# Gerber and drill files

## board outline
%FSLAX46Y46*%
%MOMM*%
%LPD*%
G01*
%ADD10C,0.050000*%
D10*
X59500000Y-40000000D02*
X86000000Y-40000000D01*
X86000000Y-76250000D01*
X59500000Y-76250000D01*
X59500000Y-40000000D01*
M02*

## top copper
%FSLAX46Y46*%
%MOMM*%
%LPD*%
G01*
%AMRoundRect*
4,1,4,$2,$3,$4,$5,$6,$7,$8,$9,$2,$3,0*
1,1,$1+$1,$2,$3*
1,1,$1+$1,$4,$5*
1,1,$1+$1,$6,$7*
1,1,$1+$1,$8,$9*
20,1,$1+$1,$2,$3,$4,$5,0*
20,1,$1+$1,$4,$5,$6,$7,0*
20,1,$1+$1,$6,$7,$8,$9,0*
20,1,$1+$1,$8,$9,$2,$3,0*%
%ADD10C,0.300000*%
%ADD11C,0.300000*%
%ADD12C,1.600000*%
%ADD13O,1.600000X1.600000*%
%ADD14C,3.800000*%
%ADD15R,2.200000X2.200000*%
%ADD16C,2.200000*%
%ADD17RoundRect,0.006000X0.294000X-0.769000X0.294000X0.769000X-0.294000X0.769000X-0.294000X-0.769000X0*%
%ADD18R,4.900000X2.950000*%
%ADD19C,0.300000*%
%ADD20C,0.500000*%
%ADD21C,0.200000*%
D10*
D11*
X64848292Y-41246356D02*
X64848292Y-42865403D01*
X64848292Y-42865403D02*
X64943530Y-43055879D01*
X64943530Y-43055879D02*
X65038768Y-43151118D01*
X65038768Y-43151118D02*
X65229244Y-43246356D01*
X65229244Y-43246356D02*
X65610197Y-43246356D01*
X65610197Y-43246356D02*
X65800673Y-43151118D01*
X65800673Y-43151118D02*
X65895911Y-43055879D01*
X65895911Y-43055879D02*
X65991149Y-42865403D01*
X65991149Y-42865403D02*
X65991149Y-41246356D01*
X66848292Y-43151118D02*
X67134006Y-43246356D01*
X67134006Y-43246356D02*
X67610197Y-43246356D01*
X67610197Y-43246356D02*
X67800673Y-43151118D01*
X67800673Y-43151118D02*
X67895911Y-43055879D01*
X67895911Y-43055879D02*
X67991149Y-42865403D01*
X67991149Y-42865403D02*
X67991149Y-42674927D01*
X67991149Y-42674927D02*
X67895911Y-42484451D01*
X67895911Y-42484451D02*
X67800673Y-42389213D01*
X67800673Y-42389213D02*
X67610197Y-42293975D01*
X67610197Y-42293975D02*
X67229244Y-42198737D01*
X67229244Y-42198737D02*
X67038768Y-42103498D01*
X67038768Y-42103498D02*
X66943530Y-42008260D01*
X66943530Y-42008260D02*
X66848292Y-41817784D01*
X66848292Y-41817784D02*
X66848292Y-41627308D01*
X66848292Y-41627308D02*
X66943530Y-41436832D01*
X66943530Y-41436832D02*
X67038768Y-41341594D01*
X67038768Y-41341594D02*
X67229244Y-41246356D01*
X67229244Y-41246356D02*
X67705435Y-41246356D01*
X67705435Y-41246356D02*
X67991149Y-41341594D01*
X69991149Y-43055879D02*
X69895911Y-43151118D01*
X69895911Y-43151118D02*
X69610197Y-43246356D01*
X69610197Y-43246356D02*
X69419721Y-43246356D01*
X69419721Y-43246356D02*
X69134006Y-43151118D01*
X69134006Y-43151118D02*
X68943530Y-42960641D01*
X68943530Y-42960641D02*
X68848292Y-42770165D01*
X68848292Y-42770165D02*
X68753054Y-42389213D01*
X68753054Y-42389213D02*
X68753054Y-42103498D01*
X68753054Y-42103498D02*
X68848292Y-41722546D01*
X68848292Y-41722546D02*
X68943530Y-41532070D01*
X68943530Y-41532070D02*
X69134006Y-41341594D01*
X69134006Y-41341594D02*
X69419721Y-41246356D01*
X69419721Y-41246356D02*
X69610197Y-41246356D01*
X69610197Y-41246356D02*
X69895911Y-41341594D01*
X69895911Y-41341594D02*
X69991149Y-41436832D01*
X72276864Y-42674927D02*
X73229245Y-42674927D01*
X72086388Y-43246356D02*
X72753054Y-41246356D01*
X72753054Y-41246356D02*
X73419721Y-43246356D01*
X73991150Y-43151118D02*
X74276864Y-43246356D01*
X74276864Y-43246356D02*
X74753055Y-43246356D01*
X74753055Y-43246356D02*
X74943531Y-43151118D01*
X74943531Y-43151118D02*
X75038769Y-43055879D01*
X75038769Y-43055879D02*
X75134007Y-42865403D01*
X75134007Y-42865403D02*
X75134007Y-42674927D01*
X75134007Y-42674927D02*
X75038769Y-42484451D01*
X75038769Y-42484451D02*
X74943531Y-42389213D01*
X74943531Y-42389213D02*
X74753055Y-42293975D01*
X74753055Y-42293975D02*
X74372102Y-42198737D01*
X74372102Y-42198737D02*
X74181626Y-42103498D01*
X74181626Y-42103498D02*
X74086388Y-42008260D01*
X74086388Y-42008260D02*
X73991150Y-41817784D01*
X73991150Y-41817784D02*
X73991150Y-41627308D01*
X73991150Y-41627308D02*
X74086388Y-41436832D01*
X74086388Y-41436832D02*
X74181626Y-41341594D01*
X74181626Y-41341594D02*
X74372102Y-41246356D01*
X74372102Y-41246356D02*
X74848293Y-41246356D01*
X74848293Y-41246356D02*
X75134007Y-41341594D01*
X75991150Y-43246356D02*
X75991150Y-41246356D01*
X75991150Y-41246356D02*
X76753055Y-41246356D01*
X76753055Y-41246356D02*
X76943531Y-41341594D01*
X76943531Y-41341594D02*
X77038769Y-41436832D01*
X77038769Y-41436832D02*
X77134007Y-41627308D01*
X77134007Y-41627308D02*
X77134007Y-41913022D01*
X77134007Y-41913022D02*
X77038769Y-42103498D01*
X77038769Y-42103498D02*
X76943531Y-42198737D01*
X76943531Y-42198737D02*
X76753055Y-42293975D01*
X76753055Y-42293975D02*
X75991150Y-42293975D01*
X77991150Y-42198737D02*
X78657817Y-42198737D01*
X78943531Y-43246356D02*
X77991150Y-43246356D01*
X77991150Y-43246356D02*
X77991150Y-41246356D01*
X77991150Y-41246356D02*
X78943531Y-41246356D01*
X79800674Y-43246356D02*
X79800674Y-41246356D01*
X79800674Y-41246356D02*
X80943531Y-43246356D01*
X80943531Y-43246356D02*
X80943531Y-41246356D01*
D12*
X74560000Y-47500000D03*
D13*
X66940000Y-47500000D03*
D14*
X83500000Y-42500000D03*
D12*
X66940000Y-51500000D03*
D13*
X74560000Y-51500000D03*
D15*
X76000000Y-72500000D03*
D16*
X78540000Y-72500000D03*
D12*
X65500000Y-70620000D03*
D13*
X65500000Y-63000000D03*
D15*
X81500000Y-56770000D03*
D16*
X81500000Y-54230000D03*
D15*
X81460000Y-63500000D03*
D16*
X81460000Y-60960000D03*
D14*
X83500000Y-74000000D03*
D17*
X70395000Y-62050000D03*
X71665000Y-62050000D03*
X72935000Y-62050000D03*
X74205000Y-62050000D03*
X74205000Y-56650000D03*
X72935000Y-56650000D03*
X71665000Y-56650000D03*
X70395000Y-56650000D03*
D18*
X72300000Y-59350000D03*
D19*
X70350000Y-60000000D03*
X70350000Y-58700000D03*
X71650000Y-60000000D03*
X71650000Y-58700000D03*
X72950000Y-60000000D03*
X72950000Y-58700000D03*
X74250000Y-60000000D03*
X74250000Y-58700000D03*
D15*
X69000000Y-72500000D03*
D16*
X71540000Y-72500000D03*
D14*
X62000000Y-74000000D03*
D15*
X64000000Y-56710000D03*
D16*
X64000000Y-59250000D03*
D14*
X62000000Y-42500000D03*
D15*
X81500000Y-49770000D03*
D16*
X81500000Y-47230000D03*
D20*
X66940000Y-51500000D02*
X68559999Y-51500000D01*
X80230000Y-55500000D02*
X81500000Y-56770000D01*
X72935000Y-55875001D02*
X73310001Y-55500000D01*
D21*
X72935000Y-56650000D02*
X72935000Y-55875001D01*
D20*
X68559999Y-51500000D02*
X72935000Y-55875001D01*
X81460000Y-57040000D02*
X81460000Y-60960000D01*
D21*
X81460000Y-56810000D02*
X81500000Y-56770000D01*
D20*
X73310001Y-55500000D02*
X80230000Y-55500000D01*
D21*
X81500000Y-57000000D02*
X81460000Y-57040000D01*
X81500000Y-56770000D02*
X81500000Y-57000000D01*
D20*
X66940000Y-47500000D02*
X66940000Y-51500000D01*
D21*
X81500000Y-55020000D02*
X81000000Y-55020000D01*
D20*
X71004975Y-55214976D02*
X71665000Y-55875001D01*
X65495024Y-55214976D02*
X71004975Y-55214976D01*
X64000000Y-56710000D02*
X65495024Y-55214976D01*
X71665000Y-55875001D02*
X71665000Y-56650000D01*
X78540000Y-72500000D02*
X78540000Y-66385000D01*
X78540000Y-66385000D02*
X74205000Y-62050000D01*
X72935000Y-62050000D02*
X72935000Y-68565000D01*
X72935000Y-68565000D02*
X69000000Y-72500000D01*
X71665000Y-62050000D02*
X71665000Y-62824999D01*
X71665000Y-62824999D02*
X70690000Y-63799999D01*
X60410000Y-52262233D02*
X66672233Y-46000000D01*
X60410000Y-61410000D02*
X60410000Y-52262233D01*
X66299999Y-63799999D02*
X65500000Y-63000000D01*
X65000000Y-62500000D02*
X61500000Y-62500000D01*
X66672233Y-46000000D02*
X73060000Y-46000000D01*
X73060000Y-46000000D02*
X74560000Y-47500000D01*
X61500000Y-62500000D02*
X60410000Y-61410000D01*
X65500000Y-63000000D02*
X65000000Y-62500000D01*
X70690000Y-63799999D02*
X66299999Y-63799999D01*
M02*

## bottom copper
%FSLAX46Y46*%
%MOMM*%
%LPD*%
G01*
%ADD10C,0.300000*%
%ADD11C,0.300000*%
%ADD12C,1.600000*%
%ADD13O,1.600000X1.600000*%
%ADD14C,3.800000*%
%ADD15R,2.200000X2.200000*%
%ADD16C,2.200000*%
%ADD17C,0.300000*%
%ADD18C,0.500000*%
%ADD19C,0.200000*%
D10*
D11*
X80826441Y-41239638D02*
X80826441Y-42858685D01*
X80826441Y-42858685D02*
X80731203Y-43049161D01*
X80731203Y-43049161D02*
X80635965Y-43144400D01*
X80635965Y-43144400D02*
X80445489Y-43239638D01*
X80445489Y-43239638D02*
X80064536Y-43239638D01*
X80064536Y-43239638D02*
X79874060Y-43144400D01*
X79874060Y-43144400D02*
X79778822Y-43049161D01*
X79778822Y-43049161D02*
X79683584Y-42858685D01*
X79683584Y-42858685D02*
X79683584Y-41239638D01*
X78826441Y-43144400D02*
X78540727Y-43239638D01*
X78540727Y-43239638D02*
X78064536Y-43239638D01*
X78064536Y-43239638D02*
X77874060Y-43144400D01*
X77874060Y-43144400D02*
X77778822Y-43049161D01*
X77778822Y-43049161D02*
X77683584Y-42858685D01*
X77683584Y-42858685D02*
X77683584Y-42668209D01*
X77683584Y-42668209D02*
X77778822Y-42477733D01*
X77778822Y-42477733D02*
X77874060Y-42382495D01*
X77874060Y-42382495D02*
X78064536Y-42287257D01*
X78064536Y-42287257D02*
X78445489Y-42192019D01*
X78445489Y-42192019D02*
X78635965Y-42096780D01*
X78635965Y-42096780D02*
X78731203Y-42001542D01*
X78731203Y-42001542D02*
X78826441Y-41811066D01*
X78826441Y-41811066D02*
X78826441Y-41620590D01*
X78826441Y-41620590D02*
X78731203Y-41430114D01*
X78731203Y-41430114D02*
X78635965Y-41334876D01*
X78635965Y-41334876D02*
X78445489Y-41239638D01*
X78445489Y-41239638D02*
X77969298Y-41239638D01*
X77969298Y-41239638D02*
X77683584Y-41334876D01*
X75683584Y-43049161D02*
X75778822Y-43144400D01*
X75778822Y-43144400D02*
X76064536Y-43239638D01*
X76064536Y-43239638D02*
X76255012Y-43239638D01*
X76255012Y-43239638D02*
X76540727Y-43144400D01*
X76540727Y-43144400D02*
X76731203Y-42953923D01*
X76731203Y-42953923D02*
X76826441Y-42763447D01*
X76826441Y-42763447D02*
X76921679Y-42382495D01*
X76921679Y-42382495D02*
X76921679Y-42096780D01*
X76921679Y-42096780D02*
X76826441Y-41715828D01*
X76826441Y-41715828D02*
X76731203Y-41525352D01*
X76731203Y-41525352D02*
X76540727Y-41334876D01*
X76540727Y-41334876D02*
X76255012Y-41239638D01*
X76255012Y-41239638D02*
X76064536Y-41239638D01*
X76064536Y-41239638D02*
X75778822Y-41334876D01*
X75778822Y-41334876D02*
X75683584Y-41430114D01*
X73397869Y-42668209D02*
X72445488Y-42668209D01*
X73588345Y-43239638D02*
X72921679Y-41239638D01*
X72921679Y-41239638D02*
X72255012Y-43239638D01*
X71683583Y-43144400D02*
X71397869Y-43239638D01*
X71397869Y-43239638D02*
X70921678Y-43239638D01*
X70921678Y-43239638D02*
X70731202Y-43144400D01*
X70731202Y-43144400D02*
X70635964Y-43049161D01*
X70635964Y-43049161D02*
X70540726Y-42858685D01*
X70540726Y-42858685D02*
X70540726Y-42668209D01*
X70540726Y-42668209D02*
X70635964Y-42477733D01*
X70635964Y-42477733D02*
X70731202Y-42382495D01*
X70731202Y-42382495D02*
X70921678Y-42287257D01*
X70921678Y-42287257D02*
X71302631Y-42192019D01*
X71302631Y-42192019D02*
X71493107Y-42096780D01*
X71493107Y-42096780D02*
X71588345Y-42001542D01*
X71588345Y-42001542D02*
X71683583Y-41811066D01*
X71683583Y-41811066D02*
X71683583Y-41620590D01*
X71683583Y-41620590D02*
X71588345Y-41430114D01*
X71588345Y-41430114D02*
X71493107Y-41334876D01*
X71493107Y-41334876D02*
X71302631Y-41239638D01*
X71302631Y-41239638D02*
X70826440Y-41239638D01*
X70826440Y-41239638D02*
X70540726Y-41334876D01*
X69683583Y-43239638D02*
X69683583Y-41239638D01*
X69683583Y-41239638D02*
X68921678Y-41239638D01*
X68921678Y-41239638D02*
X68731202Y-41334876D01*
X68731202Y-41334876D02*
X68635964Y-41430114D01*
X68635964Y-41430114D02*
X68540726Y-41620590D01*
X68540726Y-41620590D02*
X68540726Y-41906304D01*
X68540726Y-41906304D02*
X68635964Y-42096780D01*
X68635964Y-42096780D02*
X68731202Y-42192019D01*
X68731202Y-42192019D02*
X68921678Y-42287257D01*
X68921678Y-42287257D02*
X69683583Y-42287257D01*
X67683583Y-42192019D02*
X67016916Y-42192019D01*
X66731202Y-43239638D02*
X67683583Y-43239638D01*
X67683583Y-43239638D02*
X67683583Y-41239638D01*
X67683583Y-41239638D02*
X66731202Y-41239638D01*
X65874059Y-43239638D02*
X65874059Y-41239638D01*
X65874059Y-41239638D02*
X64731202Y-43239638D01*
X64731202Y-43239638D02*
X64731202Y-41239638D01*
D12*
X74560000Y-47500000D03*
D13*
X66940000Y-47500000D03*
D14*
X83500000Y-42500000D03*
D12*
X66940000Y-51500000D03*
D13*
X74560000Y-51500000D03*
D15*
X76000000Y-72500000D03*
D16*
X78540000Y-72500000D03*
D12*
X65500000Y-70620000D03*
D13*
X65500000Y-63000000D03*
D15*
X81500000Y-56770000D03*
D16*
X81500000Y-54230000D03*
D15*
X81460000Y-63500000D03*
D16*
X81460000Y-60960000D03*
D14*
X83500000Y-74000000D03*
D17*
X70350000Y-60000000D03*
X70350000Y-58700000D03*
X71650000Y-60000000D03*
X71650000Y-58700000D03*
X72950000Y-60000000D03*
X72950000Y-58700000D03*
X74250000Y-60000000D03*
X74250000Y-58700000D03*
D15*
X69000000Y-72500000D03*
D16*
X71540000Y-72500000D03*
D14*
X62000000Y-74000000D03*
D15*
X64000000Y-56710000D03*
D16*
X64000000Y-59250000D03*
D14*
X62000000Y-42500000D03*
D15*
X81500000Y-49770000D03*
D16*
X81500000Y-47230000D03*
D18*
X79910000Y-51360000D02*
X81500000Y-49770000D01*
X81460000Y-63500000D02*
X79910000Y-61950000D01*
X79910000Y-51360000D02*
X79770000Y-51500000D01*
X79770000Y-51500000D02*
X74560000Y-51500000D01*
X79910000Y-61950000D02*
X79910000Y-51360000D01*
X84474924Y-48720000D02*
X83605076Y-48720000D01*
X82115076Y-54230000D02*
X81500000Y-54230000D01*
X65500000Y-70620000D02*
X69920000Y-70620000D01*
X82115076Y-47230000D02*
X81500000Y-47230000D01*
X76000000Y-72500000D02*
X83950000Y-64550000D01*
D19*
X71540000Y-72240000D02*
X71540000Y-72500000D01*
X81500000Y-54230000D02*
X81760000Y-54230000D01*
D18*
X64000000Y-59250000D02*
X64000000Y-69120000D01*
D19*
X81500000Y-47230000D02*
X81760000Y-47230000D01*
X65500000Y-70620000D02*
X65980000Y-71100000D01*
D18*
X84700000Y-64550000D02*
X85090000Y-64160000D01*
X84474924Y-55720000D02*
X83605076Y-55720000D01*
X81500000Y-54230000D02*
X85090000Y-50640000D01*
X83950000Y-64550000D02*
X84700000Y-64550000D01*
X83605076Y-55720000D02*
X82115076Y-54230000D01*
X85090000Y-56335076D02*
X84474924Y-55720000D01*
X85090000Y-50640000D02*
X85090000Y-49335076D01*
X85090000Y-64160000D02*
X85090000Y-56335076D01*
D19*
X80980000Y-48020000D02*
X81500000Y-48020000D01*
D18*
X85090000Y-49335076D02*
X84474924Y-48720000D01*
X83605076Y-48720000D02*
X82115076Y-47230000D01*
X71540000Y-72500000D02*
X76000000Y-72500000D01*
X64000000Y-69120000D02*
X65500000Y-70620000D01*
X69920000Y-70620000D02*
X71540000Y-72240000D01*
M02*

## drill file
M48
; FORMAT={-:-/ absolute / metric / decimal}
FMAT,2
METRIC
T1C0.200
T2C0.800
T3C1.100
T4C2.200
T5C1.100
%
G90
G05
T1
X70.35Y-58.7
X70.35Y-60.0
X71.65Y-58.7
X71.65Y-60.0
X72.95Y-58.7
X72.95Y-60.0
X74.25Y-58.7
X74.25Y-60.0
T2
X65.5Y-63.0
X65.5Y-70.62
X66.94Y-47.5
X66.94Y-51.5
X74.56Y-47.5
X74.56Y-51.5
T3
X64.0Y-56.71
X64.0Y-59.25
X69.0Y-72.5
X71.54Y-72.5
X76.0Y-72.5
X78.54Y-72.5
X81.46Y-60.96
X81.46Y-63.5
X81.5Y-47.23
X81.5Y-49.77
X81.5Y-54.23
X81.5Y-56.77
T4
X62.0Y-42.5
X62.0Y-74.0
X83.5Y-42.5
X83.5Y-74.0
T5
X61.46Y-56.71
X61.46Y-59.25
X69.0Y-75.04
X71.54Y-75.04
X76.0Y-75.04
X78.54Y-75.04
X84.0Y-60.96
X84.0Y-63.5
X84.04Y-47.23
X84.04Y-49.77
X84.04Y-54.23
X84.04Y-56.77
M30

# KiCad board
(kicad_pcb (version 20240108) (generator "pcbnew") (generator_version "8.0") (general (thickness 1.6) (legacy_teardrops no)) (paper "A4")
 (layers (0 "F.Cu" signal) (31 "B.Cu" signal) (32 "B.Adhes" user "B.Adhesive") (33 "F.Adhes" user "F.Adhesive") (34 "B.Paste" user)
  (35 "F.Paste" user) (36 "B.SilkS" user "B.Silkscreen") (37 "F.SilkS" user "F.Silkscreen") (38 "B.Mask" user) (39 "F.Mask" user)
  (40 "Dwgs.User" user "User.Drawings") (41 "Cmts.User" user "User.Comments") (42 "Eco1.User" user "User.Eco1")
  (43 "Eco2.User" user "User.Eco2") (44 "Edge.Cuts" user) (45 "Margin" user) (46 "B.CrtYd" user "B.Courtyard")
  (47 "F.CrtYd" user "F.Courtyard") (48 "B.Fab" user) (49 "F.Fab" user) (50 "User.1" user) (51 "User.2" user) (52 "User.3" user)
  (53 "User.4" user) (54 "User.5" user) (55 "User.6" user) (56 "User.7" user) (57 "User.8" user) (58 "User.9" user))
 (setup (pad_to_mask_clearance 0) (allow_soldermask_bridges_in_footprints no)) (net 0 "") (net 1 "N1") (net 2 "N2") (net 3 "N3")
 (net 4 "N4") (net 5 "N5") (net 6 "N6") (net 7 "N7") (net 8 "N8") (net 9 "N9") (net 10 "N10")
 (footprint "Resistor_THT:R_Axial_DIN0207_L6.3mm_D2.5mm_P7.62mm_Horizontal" (layer "F.Cu") (at 74.56 47.5 180)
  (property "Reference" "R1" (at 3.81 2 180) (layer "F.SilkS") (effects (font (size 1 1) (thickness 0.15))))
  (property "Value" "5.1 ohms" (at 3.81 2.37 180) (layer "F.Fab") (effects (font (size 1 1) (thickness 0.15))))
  (pad "1" thru_hole circle (at 0 0 180) (size 1.6 1.6) (drill 0.8) (layers "*.Cu" "*.Mask") (remove_unused_layers no) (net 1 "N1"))
  (pad "2" thru_hole oval (at 7.62 0 180) (size 1.6 1.6) (drill 0.8) (layers "*.Cu" "*.Mask") (remove_unused_layers no) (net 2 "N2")))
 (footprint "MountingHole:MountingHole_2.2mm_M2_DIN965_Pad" (layer "F.Cu") (at 83.5 42.5)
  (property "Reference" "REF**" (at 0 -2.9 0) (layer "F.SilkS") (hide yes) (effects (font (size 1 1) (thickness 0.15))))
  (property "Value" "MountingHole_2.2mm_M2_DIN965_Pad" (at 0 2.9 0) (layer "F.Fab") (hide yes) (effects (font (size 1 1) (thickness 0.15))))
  (pad "1" thru_hole circle (at 0 0) (size 3.8 3.8) (drill 2.2) (layers "*.Cu" "*.Mask") (remove_unused_layers no)))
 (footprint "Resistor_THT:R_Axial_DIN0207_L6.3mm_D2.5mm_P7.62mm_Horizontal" (layer "F.Cu") (at 66.94 51.5)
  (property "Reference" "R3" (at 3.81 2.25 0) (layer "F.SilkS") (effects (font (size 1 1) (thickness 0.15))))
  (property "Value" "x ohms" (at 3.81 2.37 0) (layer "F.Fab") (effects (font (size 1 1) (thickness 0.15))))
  (pad "1" thru_hole circle (at 0 0) (size 1.6 1.6) (drill 0.8) (layers "*.Cu" "*.Mask") (remove_unused_layers no) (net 2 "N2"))
  (pad "2" thru_hole oval (at 7.62 0) (size 1.6 1.6) (drill 0.8) (layers "*.Cu" "*.Mask") (remove_unused_layers no) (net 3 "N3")))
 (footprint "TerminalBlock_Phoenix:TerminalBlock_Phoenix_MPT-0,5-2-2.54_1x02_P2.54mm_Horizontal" (layer "F.Cu") (at 76 72.5)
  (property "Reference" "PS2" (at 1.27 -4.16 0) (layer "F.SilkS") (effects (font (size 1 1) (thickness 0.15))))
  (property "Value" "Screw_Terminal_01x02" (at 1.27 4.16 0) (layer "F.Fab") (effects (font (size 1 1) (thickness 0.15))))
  (pad "" np_thru_hole circle (at 0 2.54) (size 1.1 1.1) (drill 1.1) (layers "*.Cu" "*.Mask"))
  (pad "" np_thru_hole circle (at 2.54 2.54) (size 1.1 1.1) (drill 1.1) (layers "*.Cu" "*.Mask"))
  (pad "1" thru_hole rect (at 0 0) (size 2.2 2.2) (drill 1.1) (layers "*.Cu" "*.Mask") (remove_unused_layers no) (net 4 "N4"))
  (pad "2" thru_hole circle (at 2.54 0) (size 2.2 2.2) (drill 1.1) (layers "*.Cu" "*.Mask") (remove_unused_layers no) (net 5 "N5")))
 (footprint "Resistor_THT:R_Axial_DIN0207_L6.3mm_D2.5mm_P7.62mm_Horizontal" (layer "F.Cu") (at 65.5 70.62 90)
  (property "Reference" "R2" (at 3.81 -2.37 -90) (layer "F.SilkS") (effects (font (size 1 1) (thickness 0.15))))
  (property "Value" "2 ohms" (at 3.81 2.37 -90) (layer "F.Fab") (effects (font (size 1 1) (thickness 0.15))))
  (pad "1" thru_hole circle (at 0 0 90) (size 1.6 1.6) (drill 0.8) (layers "*.Cu" "*.Mask") (remove_unused_layers no) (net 4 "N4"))
  (pad "2" thru_hole oval (at 7.62 0 90) (size 1.6 1.6) (drill 0.8) (layers "*.Cu" "*.Mask") (remove_unused_layers no) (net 1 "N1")))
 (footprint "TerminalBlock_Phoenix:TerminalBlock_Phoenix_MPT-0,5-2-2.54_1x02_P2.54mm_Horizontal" (layer "F.Cu") (at 81.5 56.77 90)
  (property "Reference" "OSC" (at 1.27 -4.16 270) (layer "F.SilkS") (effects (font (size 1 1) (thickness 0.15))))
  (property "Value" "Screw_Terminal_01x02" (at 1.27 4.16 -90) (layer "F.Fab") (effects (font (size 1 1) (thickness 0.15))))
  (pad "" np_thru_hole circle (at 0 2.54 90) (size 1.1 1.1) (drill 1.1) (layers "*.Cu" "*.Mask"))
  (pad "" np_thru_hole circle (at 2.54 2.54 90) (size 1.1 1.1) (drill 1.1) (layers "*.Cu" "*.Mask"))
  (pad "1" thru_hole rect (at 0 0 90) (size 2.2 2.2) (drill 1.1) (layers "*.Cu" "*.Mask") (remove_unused_layers no) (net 2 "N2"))
  (pad "2" thru_hole circle (at 2.54 0 90) (size 2.2 2.2) (drill 1.1) (layers "*.Cu" "*.Mask") (remove_unused_layers no) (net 4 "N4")))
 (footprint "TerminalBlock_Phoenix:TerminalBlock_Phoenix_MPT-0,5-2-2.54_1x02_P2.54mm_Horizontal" (layer "F.Cu") (at 81.46 63.5 90)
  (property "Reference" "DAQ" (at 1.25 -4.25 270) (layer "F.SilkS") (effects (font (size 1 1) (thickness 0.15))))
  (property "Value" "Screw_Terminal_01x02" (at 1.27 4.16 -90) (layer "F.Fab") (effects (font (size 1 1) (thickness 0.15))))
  (pad "" np_thru_hole circle (at 0 2.54 90) (size 1.1 1.1) (drill 1.1) (layers "*.Cu" "*.Mask"))
  (pad "" np_thru_hole circle (at 2.54 2.54 90) (size 1.1 1.1) (drill 1.1) (layers "*.Cu" "*.Mask"))
  (pad "1" thru_hole rect (at 0 0 90) (size 2.2 2.2) (drill 1.1) (layers "*.Cu" "*.Mask") (remove_unused_layers no) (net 3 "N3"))
  (pad "2" thru_hole circle (at 2.54 0 90) (size 2.2 2.2) (drill 1.1) (layers "*.Cu" "*.Mask") (remove_unused_layers no) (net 2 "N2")))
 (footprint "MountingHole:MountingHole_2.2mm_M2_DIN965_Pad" (layer "F.Cu") (at 83.5 74)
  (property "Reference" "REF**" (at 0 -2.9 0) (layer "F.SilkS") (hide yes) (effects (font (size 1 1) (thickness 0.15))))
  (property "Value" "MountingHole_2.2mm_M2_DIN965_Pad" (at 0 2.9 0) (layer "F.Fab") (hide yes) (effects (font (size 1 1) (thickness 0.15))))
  (pad "1" thru_hole circle (at 0 0) (size 3.8 3.8) (drill 2.2) (layers "*.Cu" "*.Mask") (remove_unused_layers no)))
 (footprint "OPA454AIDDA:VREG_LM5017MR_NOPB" (layer "F.Cu") (at 72.3 59.35 90)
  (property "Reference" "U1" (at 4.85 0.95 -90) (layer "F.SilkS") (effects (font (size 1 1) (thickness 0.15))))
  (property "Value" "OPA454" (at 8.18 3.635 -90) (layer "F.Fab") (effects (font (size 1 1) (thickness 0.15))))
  (pad "1" smd roundrect (at -2.7 -1.905 90) (size 1.55 0.6) (layers "F.Cu" "F.Paste") (roundrect_rratio 0.01) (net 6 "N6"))
  (pad "2" smd roundrect (at -2.7 -0.635 90) (size 1.55 0.6) (layers "F.Cu" "F.Paste") (roundrect_rratio 0.01) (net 1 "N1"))
  (pad "3" smd roundrect (at -2.7 0.635 90) (size 1.55 0.6) (layers "F.Cu" "F.Paste") (roundrect_rratio 0.01) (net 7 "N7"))
  (pad "4" smd roundrect (at -2.7 1.905 90) (size 1.55 0.6) (layers "F.Cu" "F.Paste") (roundrect_rratio 0.01) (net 5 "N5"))
  (pad "5" smd roundrect (at 2.7 1.905 90) (size 1.55 0.6) (layers "F.Cu" "F.Paste") (roundrect_rratio 0.01) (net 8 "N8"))
  (pad "6" smd roundrect (at 2.7 0.635 90) (size 1.55 0.6) (layers "F.Cu" "F.Paste") (roundrect_rratio 0.01) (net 2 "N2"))
  (pad "7" smd roundrect (at 2.7 -0.635 90) (size 1.55 0.6) (layers "F.Cu" "F.Paste") (roundrect_rratio 0.01) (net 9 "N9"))
  (pad "8" smd roundrect (at 2.7 -1.905 90) (size 1.55 0.6) (layers "F.Cu" "F.Paste") (roundrect_rratio 0.01) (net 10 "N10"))
  (pad "9" smd rect (at 0 0 90) (size 2.95 4.9) (layers "F.Cu"))
  (pad "10" thru_hole circle (at -0.65 -1.95 90) (size 0.3 0.3) (drill 0.2) (layers "*.Cu" "*.Mask") (remove_unused_layers no)
   (solder_mask_margin 0.102))
  (pad "11" thru_hole circle (at 0.65 -1.95 90) (size 0.3 0.3) (drill 0.2) (layers "*.Cu" "*.Mask") (remove_unused_layers no)
   (solder_mask_margin 0.102))
  (pad "12" thru_hole circle (at -0.65 -0.65 90) (size 0.3 0.3) (drill 0.2) (layers "*.Cu" "*.Mask") (remove_unused_layers no)
   (solder_mask_margin 0.102))
  (pad "13" thru_hole circle (at 0.65 -0.65 90) (size 0.3 0.3) (drill 0.2) (layers "*.Cu" "*.Mask") (remove_unused_layers no)
   (solder_mask_margin 0.102))
  (pad "14" thru_hole circle (at -0.65 0.65 90) (size 0.3 0.3) (drill 0.2) (layers "*.Cu" "*.Mask") (remove_unused_layers no)
   (solder_mask_margin 0.102))
  (pad "15" thru_hole circle (at 0.65 0.65 90) (size 0.3 0.3) (drill 0.2) (layers "*.Cu" "*.Mask") (remove_unused_layers no)
   (solder_mask_margin 0.102))
  (pad "16" thru_hole circle (at -0.65 1.95 90) (size 0.3 0.3) (drill 0.2) (layers "*.Cu" "*.Mask") (remove_unused_layers no)
   (solder_mask_margin 0.102))
  (pad "17" thru_hole circle (at 0.65 1.95 90) (size 0.3 0.3) (drill 0.2) (layers "*.Cu" "*.Mask") (remove_unused_layers no)
   (solder_mask_margin 0.102)))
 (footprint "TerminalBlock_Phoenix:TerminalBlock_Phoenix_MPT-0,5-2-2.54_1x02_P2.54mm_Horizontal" (layer "F.Cu") (at 69 72.5)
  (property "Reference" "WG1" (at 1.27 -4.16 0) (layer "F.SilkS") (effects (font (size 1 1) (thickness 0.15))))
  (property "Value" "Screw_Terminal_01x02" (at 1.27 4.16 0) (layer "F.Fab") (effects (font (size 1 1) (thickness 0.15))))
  (pad "" np_thru_hole circle (at 0 2.54) (size 1.1 1.1) (drill 1.1) (layers "*.Cu" "*.Mask"))
  (pad "" np_thru_hole circle (at 2.54 2.54) (size 1.1 1.1) (drill 1.1) (layers "*.Cu" "*.Mask"))
  (pad "1" thru_hole rect (at 0 0) (size 2.2 2.2) (drill 1.1) (layers "*.Cu" "*.Mask") (remove_unused_layers no) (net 7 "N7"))
  (pad "2" thru_hole circle (at 2.54 0) (size 2.2 2.2) (drill 1.1) (layers "*.Cu" "*.Mask") (remove_unused_layers no) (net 4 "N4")))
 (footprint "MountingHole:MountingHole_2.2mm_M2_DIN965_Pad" (layer "F.Cu") (at 62 74)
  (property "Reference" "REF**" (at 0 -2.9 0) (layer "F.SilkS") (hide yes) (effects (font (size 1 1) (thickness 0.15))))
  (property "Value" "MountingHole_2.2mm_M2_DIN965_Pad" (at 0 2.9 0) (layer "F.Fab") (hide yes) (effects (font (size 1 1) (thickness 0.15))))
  (pad "1" thru_hole circle (at 0 0) (size 3.8 3.8) (drill 2.2) (layers "*.Cu" "*.Mask") (remove_unused_layers no)))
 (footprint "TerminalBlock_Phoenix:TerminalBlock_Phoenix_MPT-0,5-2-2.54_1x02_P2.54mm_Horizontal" (layer "F.Cu") (at 64 56.71 -90)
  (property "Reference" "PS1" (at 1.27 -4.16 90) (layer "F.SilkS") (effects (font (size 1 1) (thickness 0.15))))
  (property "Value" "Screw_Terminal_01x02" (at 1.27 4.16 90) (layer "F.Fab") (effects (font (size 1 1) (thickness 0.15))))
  (pad "" np_thru_hole circle (at 0 2.54 270) (size 1.1 1.1) (drill 1.1) (layers "*.Cu" "*.Mask"))
  (pad "" np_thru_hole circle (at 2.54 2.54 270) (size 1.1 1.1) (drill 1.1) (layers "*.Cu" "*.Mask"))
  (pad "1" thru_hole rect (at 0 0 270) (size 2.2 2.2) (drill 1.1) (layers "*.Cu" "*.Mask") (remove_unused_layers no) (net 9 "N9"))
  (pad "2" thru_hole circle (at 2.54 0 270) (size 2.2 2.2) (drill 1.1) (layers "*.Cu" "*.Mask") (remove_unused_layers no) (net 4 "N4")))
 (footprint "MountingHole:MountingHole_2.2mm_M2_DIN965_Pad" (layer "F.Cu") (at 62 42.5)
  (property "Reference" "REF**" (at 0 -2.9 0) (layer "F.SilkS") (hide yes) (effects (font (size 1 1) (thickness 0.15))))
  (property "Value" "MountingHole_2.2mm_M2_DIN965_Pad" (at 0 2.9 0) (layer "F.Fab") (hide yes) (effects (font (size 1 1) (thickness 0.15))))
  (pad "1" thru_hole circle (at 0 0) (size 3.8 3.8) (drill 2.2) (layers "*.Cu" "*.Mask") (remove_unused_layers no)))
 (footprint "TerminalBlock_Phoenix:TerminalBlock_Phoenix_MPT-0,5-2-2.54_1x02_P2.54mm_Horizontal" (layer "F.Cu") (at 81.5 49.77 90)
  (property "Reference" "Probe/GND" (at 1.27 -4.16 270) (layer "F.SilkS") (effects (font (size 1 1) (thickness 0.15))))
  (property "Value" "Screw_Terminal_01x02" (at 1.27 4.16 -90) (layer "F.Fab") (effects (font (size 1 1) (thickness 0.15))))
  (pad "" np_thru_hole circle (at 0 2.54 90) (size 1.1 1.1) (drill 1.1) (layers "*.Cu" "*.Mask"))
  (pad "" np_thru_hole circle (at 2.54 2.54 90) (size 1.1 1.1) (drill 1.1) (layers "*.Cu" "*.Mask"))
  (pad "1" thru_hole rect (at 0 0 90) (size 2.2 2.2) (drill 1.1) (layers "*.Cu" "*.Mask") (remove_unused_layers no) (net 3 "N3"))
  (pad "2" thru_hole circle (at 2.54 0 90) (size 2.2 2.2) (drill 1.1) (layers "*.Cu" "*.Mask") (remove_unused_layers no) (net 4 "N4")))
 (gr_rect (start 59.5 40) (end 86 76.25) (stroke (width 0.05) (type default)) (fill none) (layer "Edge.Cuts"))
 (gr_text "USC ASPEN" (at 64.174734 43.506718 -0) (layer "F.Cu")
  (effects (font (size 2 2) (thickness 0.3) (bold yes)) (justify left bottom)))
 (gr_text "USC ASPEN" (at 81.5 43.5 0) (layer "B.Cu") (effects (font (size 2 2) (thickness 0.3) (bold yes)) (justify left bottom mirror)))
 (segment (start 79.91 51.36) (end 81.5 49.77) (width 0.5) (layer "B.Cu") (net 3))
 (segment (start 81.46 63.5) (end 79.91 61.95) (width 0.5) (layer "B.Cu") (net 3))
 (segment (start 79.91 51.36) (end 79.77 51.5) (width 0.5) (layer "B.Cu") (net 3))
 (segment (start 79.77 51.5) (end 74.56 51.5) (width 0.5) (layer "B.Cu") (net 3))
 (segment (start 79.91 61.95) (end 79.91 51.36) (width 0.5) (layer "B.Cu") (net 3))
 (segment (start 66.94 51.5) (end 68.559999 51.5) (width 0.5) (layer "F.Cu") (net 2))
 (segment (start 80.23 55.5) (end 81.5 56.77) (width 0.5) (layer "F.Cu") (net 2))
 (segment (start 72.935 55.875001) (end 73.310001 55.5) (width 0.5) (layer "F.Cu") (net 2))
 (segment (start 72.935 56.65) (end 72.935 55.875001) (width 0.2) (layer "F.Cu") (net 2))
 (segment (start 68.559999 51.5) (end 72.935 55.875001) (width 0.5) (layer "F.Cu") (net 2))
 (segment (start 81.46 57.04) (end 81.46 60.96) (width 0.5) (layer "F.Cu") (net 2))
 (segment (start 81.46 56.81) (end 81.5 56.77) (width 0.2) (layer "F.Cu") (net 2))
 (segment (start 73.310001 55.5) (end 80.23 55.5) (width 0.5) (layer "F.Cu") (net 2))
 (segment (start 81.5 57) (end 81.46 57.04) (width 0.2) (layer "F.Cu") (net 2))
 (segment (start 81.5 56.77) (end 81.5 57) (width 0.2) (layer "F.Cu") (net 2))
 (segment (start 66.94 47.5) (end 66.94 51.5) (width 0.5) (layer "F.Cu") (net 2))
 (segment (start 81.5 55.02) (end 81 55.02) (width 0.2) (layer "F.Cu") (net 4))
 (segment (start 84.474924 48.72) (end 83.605076 48.72) (width 0.5) (layer "B.Cu") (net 4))
 (segment (start 82.115076 54.23) (end 81.5 54.23) (width 0.5) (layer "B.Cu") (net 4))
 (segment (start 65.5 70.62) (end 69.92 70.62) (width 0.5) (layer "B.Cu") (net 4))
 (segment (start 82.115076 47.23) (end 81.5 47.23) (width 0.5) (layer "B.Cu") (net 4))
 (segment (start 76 72.5) (end 83.95 64.55) (width 0.5) (layer "B.Cu") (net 4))
 (segment (start 71.54 72.24) (end 71.54 72.5) (width 0.2) (layer "B.Cu") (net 4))
 (segment (start 81.5 54.23) (end 81.76 54.23) (width 0.2) (layer "B.Cu") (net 4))
 (segment (start 64 59.25) (end 64 69.12) (width 0.5) (layer "B.Cu") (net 4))
 (segment (start 81.5 47.23) (end 81.76 47.23) (width 0.2) (layer "B.Cu") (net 4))
 (segment (start 65.5 70.62) (end 65.98 71.1) (width 0.2) (layer "B.Cu") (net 4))
 (segment (start 84.7 64.55) (end 85.09 64.16) (width 0.5) (layer "B.Cu") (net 4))
 (segment (start 84.474924 55.72) (end 83.605076 55.72) (width 0.5) (layer "B.Cu") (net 4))
 (segment (start 81.5 54.23) (end 85.09 50.64) (width 0.5) (layer "B.Cu") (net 4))
 (segment (start 83.95 64.55) (end 84.7 64.55) (width 0.5) (layer "B.Cu") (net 4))
 (segment (start 83.605076 55.72) (end 82.115076 54.23) (width 0.5) (layer "B.Cu") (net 4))
 (segment (start 85.09 56.335076) (end 84.474924 55.72) (width 0.5) (layer "B.Cu") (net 4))
 (segment (start 85.09 50.64) (end 85.09 49.335076) (width 0.5) (layer "B.Cu") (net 4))
 (segment (start 85.09 64.16) (end 85.09 56.335076) (width 0.5) (layer "B.Cu") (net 4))
 (segment (start 80.98 48.02) (end 81.5 48.02) (width 0.2) (layer "B.Cu") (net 4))
 (segment (start 85.09 49.335076) (end 84.474924 48.72) (width 0.5) (layer "B.Cu") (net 4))
 (segment (start 83.605076 48.72) (end 82.115076 47.23) (width 0.5) (layer "B.Cu") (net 4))
 (segment (start 71.54 72.5) (end 76 72.5) (width 0.5) (layer "B.Cu") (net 4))
 (segment (start 64 69.12) (end 65.5 70.62) (width 0.5) (layer "B.Cu") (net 4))
 (segment (start 69.92 70.62) (end 71.54 72.24) (width 0.5) (layer "B.Cu") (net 4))
 (segment (start 71.004975 55.214976) (end 71.665 55.875001) (width 0.5) (layer "F.Cu") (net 9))
 (segment (start 65.495024 55.214976) (end 71.004975 55.214976) (width 0.5) (layer "F.Cu") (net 9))
 (segment (start 64 56.71) (end 65.495024 55.214976) (width 0.5) (layer "F.Cu") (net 9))
 (segment (start 71.665 55.875001) (end 71.665 56.65) (width 0.5) (layer "F.Cu") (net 9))
 (segment (start 78.54 72.5) (end 78.54 66.385) (width 0.5) (layer "F.Cu") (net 5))
 (segment (start 78.54 66.385) (end 74.205 62.05) (width 0.5) (layer "F.Cu") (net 5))
 (segment (start 72.935 62.05) (end 72.935 68.565) (width 0.5) (layer "F.Cu") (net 7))
 (segment (start 72.935 68.565) (end 69 72.5) (width 0.5) (layer "F.Cu") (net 7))
 (segment (start 71.665 62.05) (end 71.665 62.824999) (width 0.5) (layer "F.Cu") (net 1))
 (segment (start 71.665 62.824999) (end 70.69 63.799999) (width 0.5) (layer "F.Cu") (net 1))
 (segment (start 60.41 52.262233) (end 66.672233 46) (width 0.5) (layer "F.Cu") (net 1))
 (segment (start 60.41 61.41) (end 60.41 52.262233) (width 0.5) (layer "F.Cu") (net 1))
 (segment (start 66.299999 63.799999) (end 65.5 63) (width 0.5) (layer "F.Cu") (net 1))
 (segment (start 65 62.5) (end 61.5 62.5) (width 0.5) (layer "F.Cu") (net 1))
 (segment (start 66.672233 46) (end 73.06 46) (width 0.5) (layer "F.Cu") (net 1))
 (segment (start 73.06 46) (end 74.56 47.5) (width 0.5) (layer "F.Cu") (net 1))
 (segment (start 61.5 62.5) (end 60.41 61.41) (width 0.5) (layer "F.Cu") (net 1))
 (segment (start 65.5 63) (end 65 62.5) (width 0.5) (layer "F.Cu") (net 1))
 (segment (start 70.69 63.799999) (end 66.299999 63.799999) (width 0.5) (layer "F.Cu") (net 1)))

